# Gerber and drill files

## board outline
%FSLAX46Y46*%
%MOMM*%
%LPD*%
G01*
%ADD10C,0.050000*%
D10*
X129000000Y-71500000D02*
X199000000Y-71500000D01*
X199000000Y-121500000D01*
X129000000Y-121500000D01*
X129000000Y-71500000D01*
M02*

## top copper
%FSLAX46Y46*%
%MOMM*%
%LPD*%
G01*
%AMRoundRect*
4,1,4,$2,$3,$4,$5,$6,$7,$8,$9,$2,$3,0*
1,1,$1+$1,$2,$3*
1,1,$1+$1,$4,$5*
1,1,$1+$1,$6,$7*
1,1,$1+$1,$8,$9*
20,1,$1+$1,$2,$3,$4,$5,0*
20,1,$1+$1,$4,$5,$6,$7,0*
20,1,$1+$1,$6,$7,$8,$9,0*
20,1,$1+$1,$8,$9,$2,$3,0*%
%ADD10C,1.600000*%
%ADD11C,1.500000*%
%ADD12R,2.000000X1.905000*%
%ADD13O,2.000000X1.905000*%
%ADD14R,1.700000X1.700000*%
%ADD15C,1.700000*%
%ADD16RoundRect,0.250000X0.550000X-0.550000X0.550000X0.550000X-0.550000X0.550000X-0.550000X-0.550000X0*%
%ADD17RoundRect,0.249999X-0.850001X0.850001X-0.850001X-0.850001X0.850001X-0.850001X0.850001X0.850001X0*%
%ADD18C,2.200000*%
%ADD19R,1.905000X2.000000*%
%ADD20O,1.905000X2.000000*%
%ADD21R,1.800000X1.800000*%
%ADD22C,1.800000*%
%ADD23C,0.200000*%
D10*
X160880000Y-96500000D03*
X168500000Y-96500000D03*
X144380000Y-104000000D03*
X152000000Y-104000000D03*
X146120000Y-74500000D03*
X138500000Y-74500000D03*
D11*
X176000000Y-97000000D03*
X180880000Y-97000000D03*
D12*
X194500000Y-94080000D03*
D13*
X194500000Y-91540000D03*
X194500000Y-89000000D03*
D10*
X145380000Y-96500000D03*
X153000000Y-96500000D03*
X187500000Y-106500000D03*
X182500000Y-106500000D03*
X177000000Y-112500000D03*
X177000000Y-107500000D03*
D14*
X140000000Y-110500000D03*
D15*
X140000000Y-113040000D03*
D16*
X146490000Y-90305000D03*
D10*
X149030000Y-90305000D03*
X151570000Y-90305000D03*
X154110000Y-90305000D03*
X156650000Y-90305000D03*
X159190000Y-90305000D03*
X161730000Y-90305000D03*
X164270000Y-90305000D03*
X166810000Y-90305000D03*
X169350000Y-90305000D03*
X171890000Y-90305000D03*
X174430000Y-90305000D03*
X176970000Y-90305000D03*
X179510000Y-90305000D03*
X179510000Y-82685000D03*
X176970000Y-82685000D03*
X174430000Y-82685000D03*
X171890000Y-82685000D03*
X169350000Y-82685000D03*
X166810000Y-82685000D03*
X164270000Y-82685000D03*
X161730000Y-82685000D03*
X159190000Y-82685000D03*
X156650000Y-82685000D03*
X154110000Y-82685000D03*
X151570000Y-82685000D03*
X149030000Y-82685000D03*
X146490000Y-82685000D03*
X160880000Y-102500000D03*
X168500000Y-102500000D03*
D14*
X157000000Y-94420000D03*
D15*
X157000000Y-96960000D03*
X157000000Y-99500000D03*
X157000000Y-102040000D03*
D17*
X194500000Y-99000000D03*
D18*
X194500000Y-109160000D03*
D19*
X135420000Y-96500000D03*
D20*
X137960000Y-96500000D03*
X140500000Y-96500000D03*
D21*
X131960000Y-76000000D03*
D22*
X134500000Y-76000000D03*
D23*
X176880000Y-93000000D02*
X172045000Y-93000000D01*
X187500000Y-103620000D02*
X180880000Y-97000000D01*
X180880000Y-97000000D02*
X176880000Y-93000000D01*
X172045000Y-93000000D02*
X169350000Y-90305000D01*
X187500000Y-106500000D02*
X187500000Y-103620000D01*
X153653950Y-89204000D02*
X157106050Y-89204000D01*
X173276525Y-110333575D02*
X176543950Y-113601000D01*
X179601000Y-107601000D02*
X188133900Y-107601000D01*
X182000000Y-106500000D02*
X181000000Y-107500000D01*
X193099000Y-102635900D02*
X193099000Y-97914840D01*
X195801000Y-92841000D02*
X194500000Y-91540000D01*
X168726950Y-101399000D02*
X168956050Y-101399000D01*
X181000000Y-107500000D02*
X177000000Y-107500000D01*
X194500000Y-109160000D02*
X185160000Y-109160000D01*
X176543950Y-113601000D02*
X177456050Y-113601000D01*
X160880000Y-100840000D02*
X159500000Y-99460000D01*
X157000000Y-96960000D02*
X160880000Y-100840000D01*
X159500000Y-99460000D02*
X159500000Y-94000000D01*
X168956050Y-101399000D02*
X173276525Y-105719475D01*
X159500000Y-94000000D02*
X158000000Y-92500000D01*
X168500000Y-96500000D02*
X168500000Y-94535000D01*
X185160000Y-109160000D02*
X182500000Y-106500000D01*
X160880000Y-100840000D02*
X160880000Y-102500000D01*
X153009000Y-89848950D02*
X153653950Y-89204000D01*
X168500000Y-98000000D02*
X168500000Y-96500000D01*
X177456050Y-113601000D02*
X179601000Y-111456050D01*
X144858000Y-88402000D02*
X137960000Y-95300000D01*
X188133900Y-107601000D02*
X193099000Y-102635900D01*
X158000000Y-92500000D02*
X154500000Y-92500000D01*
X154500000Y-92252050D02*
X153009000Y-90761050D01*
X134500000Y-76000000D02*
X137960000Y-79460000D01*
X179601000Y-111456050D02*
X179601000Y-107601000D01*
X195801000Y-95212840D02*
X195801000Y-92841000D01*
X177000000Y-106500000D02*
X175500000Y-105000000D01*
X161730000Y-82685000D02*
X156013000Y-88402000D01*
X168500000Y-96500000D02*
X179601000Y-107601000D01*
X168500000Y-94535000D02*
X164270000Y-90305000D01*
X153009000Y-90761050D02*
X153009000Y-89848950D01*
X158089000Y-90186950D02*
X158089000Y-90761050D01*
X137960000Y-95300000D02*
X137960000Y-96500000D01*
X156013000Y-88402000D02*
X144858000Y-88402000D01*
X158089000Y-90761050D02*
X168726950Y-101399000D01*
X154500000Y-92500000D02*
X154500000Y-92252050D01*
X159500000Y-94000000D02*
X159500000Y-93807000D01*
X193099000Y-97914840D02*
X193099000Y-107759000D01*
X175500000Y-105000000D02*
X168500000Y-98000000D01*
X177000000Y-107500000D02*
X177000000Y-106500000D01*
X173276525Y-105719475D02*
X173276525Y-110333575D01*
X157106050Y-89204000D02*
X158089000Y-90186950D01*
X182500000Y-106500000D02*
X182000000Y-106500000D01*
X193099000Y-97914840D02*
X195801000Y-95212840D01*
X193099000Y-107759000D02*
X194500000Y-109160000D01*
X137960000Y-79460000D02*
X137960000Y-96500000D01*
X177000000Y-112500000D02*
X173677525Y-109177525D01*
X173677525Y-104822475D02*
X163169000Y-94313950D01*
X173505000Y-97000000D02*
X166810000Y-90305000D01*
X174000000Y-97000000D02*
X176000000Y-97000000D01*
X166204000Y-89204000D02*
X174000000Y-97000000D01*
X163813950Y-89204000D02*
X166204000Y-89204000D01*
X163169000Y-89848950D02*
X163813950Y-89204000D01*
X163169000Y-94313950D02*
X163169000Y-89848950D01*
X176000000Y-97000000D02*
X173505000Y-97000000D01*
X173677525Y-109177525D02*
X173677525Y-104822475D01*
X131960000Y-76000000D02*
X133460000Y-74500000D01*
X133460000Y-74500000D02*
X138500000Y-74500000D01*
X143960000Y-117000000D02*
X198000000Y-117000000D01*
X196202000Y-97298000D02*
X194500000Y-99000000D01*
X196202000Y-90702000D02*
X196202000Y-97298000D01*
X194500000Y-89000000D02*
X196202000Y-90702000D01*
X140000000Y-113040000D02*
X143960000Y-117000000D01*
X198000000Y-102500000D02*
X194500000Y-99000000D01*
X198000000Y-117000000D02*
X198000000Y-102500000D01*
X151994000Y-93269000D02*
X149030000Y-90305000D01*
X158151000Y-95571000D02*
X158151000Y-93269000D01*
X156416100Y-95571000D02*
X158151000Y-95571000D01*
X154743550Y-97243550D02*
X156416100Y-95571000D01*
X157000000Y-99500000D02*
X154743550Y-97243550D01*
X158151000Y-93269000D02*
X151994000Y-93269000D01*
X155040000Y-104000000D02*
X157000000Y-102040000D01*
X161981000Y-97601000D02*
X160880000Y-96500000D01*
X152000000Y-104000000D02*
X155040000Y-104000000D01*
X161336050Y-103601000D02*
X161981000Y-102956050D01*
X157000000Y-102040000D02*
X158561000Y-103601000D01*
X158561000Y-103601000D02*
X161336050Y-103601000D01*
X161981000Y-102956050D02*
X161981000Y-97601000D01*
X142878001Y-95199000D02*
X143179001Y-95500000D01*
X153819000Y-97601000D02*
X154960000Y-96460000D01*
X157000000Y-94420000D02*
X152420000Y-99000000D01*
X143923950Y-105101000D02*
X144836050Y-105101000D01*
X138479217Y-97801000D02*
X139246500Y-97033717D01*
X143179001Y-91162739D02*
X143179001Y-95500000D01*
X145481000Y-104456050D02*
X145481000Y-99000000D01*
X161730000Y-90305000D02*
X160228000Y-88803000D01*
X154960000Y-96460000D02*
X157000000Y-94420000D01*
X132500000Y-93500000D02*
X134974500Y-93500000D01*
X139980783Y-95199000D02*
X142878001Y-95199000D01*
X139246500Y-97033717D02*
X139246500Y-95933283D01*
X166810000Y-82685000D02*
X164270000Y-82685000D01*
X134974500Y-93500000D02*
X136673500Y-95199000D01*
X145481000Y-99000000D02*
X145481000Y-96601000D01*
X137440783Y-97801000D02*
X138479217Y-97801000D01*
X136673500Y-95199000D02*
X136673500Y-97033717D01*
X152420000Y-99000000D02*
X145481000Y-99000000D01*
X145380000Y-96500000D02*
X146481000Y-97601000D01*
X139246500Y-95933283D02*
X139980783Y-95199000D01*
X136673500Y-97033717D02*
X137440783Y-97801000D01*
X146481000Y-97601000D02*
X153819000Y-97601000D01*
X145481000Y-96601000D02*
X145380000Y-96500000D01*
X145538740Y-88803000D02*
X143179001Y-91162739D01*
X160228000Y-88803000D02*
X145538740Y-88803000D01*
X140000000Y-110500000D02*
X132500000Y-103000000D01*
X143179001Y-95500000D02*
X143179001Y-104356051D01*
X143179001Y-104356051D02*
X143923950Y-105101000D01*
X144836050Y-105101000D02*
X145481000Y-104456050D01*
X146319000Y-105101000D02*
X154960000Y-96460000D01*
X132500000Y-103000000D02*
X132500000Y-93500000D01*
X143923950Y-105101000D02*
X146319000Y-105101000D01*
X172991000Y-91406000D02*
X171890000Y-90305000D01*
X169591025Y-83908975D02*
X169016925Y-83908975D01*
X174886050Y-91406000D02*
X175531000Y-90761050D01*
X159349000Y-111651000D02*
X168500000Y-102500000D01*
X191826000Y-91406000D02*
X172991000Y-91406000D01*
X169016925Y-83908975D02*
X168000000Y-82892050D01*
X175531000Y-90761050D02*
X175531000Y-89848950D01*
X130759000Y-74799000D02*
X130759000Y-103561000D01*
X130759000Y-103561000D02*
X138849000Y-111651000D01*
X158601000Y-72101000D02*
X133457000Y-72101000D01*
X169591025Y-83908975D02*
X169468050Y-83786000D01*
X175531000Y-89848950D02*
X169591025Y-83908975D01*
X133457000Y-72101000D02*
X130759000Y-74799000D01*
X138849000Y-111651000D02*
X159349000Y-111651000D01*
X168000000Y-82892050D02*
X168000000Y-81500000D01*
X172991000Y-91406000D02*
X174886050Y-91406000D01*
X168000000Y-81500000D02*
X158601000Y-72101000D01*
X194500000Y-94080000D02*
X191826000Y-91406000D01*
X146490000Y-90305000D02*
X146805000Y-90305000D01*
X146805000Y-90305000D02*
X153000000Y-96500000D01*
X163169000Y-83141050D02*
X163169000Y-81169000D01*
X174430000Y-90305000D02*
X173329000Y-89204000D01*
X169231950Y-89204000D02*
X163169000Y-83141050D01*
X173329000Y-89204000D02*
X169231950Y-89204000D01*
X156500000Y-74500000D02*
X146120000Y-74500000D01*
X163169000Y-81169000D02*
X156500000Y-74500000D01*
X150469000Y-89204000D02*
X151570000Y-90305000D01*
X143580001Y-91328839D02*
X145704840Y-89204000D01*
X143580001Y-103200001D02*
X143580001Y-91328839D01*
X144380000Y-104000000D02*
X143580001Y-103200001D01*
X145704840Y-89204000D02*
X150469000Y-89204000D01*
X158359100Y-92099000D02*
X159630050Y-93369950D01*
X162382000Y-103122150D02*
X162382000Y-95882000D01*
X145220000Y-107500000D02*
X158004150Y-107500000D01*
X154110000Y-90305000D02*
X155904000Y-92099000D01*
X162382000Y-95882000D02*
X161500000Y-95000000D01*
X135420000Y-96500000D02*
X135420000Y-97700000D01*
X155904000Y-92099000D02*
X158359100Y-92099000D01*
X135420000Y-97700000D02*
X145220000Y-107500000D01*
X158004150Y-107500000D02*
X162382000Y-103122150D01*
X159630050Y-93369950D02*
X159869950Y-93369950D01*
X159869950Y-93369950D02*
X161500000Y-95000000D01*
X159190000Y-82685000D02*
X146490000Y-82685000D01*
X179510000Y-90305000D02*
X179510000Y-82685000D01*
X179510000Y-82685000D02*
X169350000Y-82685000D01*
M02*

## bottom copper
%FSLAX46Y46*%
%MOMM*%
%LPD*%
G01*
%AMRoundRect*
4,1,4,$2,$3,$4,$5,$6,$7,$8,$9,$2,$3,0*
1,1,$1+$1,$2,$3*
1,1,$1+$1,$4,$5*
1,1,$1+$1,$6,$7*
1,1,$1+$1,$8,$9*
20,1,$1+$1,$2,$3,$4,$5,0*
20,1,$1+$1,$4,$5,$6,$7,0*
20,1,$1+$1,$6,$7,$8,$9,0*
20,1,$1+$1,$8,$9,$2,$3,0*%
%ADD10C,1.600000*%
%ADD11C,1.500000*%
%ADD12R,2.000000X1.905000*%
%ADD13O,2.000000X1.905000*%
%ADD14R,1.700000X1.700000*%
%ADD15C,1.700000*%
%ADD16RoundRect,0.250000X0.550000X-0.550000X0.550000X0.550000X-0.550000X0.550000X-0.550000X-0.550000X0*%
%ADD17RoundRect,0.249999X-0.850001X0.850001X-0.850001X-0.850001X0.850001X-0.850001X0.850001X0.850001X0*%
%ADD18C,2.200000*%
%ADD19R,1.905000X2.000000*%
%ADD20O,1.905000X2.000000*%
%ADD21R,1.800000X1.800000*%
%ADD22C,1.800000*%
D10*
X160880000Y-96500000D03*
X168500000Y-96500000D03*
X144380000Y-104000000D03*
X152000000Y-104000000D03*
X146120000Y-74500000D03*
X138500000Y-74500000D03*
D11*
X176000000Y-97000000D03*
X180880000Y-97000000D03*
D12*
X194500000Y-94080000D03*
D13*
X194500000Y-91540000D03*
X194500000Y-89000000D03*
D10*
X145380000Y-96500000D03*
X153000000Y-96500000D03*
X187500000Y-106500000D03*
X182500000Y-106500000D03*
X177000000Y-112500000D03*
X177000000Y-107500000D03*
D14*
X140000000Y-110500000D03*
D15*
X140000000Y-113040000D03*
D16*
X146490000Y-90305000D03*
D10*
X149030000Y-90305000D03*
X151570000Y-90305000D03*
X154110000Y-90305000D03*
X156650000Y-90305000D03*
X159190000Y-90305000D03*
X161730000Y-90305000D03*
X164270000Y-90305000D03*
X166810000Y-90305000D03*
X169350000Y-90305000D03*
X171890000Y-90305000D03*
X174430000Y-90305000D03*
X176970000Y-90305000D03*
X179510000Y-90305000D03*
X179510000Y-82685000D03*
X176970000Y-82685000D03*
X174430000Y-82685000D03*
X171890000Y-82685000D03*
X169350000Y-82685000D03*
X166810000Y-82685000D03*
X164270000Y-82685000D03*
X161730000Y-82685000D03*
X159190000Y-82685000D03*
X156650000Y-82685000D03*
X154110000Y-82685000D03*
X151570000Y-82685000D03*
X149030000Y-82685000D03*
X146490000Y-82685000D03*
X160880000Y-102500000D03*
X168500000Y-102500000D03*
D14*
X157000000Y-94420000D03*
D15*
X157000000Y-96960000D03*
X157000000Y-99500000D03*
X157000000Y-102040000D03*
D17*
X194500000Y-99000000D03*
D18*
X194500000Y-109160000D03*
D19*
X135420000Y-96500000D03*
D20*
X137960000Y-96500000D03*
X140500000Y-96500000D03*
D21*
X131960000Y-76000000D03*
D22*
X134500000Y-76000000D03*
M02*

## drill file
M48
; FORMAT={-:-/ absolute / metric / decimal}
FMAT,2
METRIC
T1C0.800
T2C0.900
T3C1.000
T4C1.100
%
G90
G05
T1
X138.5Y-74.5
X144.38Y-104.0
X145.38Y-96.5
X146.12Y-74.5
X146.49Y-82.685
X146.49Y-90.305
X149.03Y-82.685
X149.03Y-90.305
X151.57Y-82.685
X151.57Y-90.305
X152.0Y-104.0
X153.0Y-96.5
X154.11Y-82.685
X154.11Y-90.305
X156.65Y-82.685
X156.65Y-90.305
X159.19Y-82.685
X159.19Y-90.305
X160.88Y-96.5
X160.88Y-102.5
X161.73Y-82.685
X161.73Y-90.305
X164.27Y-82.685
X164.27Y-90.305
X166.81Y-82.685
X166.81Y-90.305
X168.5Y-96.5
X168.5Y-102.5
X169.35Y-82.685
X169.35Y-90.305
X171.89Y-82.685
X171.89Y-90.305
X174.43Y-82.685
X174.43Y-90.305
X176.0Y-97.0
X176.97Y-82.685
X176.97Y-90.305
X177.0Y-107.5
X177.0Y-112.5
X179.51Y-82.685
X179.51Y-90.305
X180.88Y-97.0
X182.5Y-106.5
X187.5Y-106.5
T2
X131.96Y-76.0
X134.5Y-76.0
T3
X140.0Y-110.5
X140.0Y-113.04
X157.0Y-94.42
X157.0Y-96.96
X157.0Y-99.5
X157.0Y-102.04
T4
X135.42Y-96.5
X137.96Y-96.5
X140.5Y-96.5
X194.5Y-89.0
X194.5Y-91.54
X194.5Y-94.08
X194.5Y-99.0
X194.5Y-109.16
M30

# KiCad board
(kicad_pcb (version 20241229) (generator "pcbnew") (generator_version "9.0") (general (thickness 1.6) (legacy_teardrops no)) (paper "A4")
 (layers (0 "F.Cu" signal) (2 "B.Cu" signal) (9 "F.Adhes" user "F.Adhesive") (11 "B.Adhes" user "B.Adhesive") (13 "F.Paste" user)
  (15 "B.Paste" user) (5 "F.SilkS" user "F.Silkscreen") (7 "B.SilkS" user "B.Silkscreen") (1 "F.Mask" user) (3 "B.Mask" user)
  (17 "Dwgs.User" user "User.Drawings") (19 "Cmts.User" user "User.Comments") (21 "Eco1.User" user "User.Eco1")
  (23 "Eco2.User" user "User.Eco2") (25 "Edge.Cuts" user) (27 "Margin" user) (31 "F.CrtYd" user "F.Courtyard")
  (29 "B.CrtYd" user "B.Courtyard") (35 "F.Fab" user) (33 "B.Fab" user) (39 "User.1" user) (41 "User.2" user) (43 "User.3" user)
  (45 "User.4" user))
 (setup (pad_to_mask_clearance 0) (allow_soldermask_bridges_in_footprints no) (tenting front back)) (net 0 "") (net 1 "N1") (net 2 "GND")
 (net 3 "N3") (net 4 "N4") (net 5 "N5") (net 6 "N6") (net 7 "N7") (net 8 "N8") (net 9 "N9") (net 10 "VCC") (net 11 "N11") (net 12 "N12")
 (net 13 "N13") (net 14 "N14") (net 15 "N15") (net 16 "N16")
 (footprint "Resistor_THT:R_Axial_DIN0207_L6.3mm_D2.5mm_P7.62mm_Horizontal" (layer "F.Cu") (at 160.88 96.5)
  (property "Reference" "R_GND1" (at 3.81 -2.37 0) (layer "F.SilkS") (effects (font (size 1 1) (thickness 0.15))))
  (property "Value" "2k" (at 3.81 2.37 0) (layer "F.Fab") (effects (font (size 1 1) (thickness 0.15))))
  (pad "1" thru_hole circle (at 0 0) (size 1.6 1.6) (drill 0.8) (layers "*.Cu" "*.Mask") (remove_unused_layers no) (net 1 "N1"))
  (pad "2" thru_hole circle (at 7.62 0) (size 1.6 1.6) (drill 0.8) (layers "*.Cu" "*.Mask") (remove_unused_layers no) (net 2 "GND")))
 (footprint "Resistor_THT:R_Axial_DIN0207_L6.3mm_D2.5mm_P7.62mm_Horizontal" (layer "F.Cu") (at 144.38 104)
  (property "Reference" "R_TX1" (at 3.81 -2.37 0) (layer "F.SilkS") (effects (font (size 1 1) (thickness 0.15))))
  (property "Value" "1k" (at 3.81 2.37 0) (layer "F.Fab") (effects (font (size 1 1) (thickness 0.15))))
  (pad "1" thru_hole circle (at 0 0) (size 1.6 1.6) (drill 0.8) (layers "*.Cu" "*.Mask") (remove_unused_layers no) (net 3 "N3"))
  (pad "2" thru_hole circle (at 7.62 0) (size 1.6 1.6) (drill 0.8) (layers "*.Cu" "*.Mask") (remove_unused_layers no) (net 1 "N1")))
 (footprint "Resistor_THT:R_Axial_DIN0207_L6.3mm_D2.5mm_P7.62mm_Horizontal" (layer "F.Cu") (at 146.12 74.5 180)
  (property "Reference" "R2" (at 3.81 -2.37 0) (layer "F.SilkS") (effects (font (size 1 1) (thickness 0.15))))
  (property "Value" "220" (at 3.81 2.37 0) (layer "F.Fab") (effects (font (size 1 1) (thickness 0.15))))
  (pad "1" thru_hole circle (at 0 0 180) (size 1.6 1.6) (drill 0.8) (layers "*.Cu" "*.Mask") (remove_unused_layers no) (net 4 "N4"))
  (pad "2" thru_hole circle (at 7.62 0 180) (size 1.6 1.6) (drill 0.8) (layers "*.Cu" "*.Mask") (remove_unused_layers no) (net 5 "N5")))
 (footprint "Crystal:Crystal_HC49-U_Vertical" (layer "F.Cu") (at 176 97)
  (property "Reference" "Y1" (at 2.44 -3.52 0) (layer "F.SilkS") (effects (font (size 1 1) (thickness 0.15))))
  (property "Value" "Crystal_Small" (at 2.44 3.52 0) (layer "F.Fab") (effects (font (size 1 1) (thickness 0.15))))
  (pad "1" thru_hole circle (at 0 0) (size 1.5 1.5) (drill 0.8) (layers "*.Cu" "*.Mask") (remove_unused_layers no) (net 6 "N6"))
  (pad "2" thru_hole circle (at 4.88 0) (size 1.5 1.5) (drill 0.8) (layers "*.Cu" "*.Mask") (remove_unused_layers no) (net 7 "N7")))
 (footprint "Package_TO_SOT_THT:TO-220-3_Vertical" (layer "F.Cu") (at 194.5 94.08 90)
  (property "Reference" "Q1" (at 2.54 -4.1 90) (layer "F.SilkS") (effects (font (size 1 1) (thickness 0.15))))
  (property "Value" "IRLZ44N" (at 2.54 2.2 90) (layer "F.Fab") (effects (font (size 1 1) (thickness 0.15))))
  (pad "1" thru_hole rect (at 0 0 90) (size 1.905 2) (drill 1.1) (layers "*.Cu" "*.Mask") (remove_unused_layers no) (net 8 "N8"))
  (pad "2" thru_hole oval (at 2.54 0 90) (size 1.905 2) (drill 1.1) (layers "*.Cu" "*.Mask") (remove_unused_layers no) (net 2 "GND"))
  (pad "3" thru_hole oval (at 5.08 0 90) (size 1.905 2) (drill 1.1) (layers "*.Cu" "*.Mask") (remove_unused_layers no) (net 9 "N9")))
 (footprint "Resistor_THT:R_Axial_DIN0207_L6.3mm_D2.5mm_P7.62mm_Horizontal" (layer "F.Cu") (at 145.38 96.5)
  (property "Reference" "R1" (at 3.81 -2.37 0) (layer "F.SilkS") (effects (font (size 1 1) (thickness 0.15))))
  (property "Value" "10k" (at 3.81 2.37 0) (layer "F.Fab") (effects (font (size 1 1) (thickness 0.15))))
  (pad "1" thru_hole circle (at 0 0) (size 1.6 1.6) (drill 0.8) (layers "*.Cu" "*.Mask") (remove_unused_layers no) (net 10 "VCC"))
  (pad "2" thru_hole circle (at 7.62 0) (size 1.6 1.6) (drill 0.8) (layers "*.Cu" "*.Mask") (remove_unused_layers no) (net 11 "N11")))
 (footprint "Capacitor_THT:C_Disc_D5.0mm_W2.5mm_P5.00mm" (layer "F.Cu") (at 187.5 106.5 180)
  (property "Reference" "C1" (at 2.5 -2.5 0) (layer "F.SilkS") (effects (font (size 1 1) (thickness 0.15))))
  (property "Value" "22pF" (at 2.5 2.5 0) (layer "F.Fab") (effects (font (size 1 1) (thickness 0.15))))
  (pad "1" thru_hole circle (at 0 0 180) (size 1.6 1.6) (drill 0.8) (layers "*.Cu" "*.Mask") (remove_unused_layers no) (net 7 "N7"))
  (pad "2" thru_hole circle (at 5 0 180) (size 1.6 1.6) (drill 0.8) (layers "*.Cu" "*.Mask") (remove_unused_layers no) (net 2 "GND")))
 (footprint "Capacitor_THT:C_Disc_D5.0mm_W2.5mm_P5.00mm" (layer "F.Cu") (at 177 112.5 90)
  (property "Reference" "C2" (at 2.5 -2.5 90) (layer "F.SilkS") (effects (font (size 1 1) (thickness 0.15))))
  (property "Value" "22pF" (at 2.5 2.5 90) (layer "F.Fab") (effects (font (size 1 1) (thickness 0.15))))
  (pad "1" thru_hole circle (at 0 0 90) (size 1.6 1.6) (drill 0.8) (layers "*.Cu" "*.Mask") (remove_unused_layers no) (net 6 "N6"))
  (pad "2" thru_hole circle (at 5 0 90) (size 1.6 1.6) (drill 0.8) (layers "*.Cu" "*.Mask") (remove_unused_layers no) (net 2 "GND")))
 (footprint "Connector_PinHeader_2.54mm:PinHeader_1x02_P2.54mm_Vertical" (layer "F.Cu") (at 140 110.5)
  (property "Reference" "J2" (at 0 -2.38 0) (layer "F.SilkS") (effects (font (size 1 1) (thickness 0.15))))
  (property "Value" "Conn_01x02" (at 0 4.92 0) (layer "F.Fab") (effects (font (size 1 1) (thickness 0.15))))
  (pad "1" thru_hole rect (at 0 0) (size 1.7 1.7) (drill 1) (layers "*.Cu" "*.Mask") (remove_unused_layers no) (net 10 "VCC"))
  (pad "2" thru_hole circle (at 0 2.54) (size 1.7 1.7) (drill 1) (layers "*.Cu" "*.Mask") (remove_unused_layers no) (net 9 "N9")))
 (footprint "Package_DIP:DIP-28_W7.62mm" (layer "F.Cu") (at 146.49 90.305 90)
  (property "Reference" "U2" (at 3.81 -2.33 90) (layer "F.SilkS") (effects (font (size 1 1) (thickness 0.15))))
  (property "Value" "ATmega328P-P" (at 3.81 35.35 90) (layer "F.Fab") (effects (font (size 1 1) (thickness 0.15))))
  (pad "1" thru_hole roundrect (at 0 0 90) (size 1.6 1.6) (drill 0.8) (layers "*.Cu" "*.Mask") (remove_unused_layers no)
   (roundrect_rratio 0.15625) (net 11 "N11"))
  (pad "2" thru_hole circle (at 0 2.54 90) (size 1.6 1.6) (drill 0.8) (layers "*.Cu" "*.Mask") (remove_unused_layers no) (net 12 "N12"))
  (pad "3" thru_hole circle (at 0 5.08 90) (size 1.6 1.6) (drill 0.8) (layers "*.Cu" "*.Mask") (remove_unused_layers no) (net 3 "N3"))
  (pad "4" thru_hole circle (at 0 7.62 90) (size 1.6 1.6) (drill 0.8) (layers "*.Cu" "*.Mask") (remove_unused_layers no) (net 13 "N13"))
  (pad "5" thru_hole circle (at 0 10.16 90) (size 1.6 1.6) (drill 0.8) (layers "*.Cu" "*.Mask") (remove_unused_layers no) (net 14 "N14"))
  (pad "6" thru_hole circle (at 0 12.7 90) (size 1.6 1.6) (drill 0.8) (layers "*.Cu" "*.Mask") (remove_unused_layers no) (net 14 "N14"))
  (pad "7" thru_hole circle (at 0 15.24 90) (size 1.6 1.6) (drill 0.8) (layers "*.Cu" "*.Mask") (remove_unused_layers no) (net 10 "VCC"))
  (pad "8" thru_hole circle (at 0 17.78 90) (size 1.6 1.6) (drill 0.8) (layers "*.Cu" "*.Mask") (remove_unused_layers no) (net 2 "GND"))
  (pad "9" thru_hole circle (at 0 20.32 90) (size 1.6 1.6) (drill 0.8) (layers "*.Cu" "*.Mask") (remove_unused_layers no) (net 6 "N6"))
  (pad "10" thru_hole circle (at 0 22.86 90) (size 1.6 1.6) (drill 0.8) (layers "*.Cu" "*.Mask") (remove_unused_layers no) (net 7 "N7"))
  (pad "11" thru_hole circle (at 0 25.4 90) (size 1.6 1.6) (drill 0.8) (layers "*.Cu" "*.Mask") (remove_unused_layers no) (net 8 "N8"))
  (pad "12" thru_hole circle (at 0 27.94 90) (size 1.6 1.6) (drill 0.8) (layers "*.Cu" "*.Mask") (remove_unused_layers no) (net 4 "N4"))
  (pad "13" thru_hole circle (at 0 30.48 90) (size 1.6 1.6) (drill 0.8) (layers "*.Cu" "*.Mask") (remove_unused_layers no) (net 14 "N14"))
  (pad "14" thru_hole circle (at 0 33.02 90) (size 1.6 1.6) (drill 0.8) (layers "*.Cu" "*.Mask") (remove_unused_layers no) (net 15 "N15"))
  (pad "15" thru_hole circle (at 7.62 33.02 90) (size 1.6 1.6) (drill 0.8) (layers "*.Cu" "*.Mask") (remove_unused_layers no) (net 15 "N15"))
  (pad "16" thru_hole circle (at 7.62 30.48 90) (size 1.6 1.6) (drill 0.8) (layers "*.Cu" "*.Mask") (remove_unused_layers no) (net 15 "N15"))
  (pad "17" thru_hole circle (at 7.62 27.94 90) (size 1.6 1.6) (drill 0.8) (layers "*.Cu" "*.Mask") (remove_unused_layers no) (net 15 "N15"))
  (pad "18" thru_hole circle (at 7.62 25.4 90) (size 1.6 1.6) (drill 0.8) (layers "*.Cu" "*.Mask") (remove_unused_layers no) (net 15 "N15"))
  (pad "19" thru_hole circle (at 7.62 22.86 90) (size 1.6 1.6) (drill 0.8) (layers "*.Cu" "*.Mask") (remove_unused_layers no) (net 15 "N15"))
  (pad "20" thru_hole circle (at 7.62 20.32 90) (size 1.6 1.6) (drill 0.8) (layers "*.Cu" "*.Mask") (remove_unused_layers no) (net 10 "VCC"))
  (pad "21" thru_hole circle (at 7.62 17.78 90) (size 1.6 1.6) (drill 0.8) (layers "*.Cu" "*.Mask") (remove_unused_layers no) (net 10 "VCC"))
  (pad "22" thru_hole circle (at 7.62 15.24 90) (size 1.6 1.6) (drill 0.8) (layers "*.Cu" "*.Mask") (remove_unused_layers no) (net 2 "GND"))
  (pad "23" thru_hole circle (at 7.62 12.7 90) (size 1.6 1.6) (drill 0.8) (layers "*.Cu" "*.Mask") (remove_unused_layers no) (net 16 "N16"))
  (pad "24" thru_hole circle (at 7.62 10.16 90) (size 1.6 1.6) (drill 0.8) (layers "*.Cu" "*.Mask") (remove_unused_layers no) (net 16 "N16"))
  (pad "25" thru_hole circle (at 7.62 7.62 90) (size 1.6 1.6) (drill 0.8) (layers "*.Cu" "*.Mask") (remove_unused_layers no) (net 16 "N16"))
  (pad "26" thru_hole circle (at 7.62 5.08 90) (size 1.6 1.6) (drill 0.8) (layers "*.Cu" "*.Mask") (remove_unused_layers no) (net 16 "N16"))
  (pad "27" thru_hole circle (at 7.62 2.54 90) (size 1.6 1.6) (drill 0.8) (layers "*.Cu" "*.Mask") (remove_unused_layers no) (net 16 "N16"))
  (pad "28" thru_hole circle (at 7.62 0 90) (size 1.6 1.6) (drill 0.8) (layers "*.Cu" "*.Mask") (remove_unused_layers no) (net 16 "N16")))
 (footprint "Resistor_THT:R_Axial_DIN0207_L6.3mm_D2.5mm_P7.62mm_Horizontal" (layer "F.Cu") (at 160.88 102.5)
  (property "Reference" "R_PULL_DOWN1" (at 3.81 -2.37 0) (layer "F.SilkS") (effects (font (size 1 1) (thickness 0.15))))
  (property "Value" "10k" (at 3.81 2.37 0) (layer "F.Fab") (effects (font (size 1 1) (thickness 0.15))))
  (pad "1" thru_hole circle (at 0 0) (size 1.6 1.6) (drill 0.8) (layers "*.Cu" "*.Mask") (remove_unused_layers no) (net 2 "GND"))
  (pad "2" thru_hole circle (at 7.62 0) (size 1.6 1.6) (drill 0.8) (layers "*.Cu" "*.Mask") (remove_unused_layers no) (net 8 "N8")))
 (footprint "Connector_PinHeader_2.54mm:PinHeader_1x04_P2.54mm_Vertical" (layer "F.Cu") (at 157 94.42)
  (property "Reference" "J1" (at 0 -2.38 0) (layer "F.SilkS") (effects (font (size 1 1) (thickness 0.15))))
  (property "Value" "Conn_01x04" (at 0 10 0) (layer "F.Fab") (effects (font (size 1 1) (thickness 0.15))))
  (pad "1" thru_hole rect (at 0 0) (size 1.7 1.7) (drill 1) (layers "*.Cu" "*.Mask") (remove_unused_layers no) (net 10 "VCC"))
  (pad "2" thru_hole circle (at 0 2.54) (size 1.7 1.7) (drill 1) (layers "*.Cu" "*.Mask") (remove_unused_layers no) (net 2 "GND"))
  (pad "3" thru_hole circle (at 0 5.08) (size 1.7 1.7) (drill 1) (layers "*.Cu" "*.Mask") (remove_unused_layers no) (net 12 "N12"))
  (pad "4" thru_hole circle (at 0 7.62) (size 1.7 1.7) (drill 1) (layers "*.Cu" "*.Mask") (remove_unused_layers no) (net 1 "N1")))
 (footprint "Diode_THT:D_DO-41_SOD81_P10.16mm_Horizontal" (layer "F.Cu") (at 194.5 99 -90)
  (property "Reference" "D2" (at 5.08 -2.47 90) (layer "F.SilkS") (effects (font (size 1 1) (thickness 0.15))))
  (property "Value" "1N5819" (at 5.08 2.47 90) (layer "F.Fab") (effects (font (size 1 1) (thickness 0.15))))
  (pad "1" thru_hole roundrect (at 0 0 270) (size 2.2 2.2) (drill 1.1) (layers "*.Cu" "*.Mask") (remove_unused_layers no)
   (roundrect_rratio 0.113636) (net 9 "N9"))
  (pad "2" thru_hole circle (at 10.16 0 270) (size 2.2 2.2) (drill 1.1) (layers "*.Cu" "*.Mask") (remove_unused_layers no) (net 2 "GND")))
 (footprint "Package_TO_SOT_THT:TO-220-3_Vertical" (layer "F.Cu") (at 135.42 96.5)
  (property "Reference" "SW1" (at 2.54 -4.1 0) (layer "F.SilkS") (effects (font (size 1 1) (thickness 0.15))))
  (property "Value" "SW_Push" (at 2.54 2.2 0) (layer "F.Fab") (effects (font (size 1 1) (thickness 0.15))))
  (pad "1" thru_hole rect (at 0 0) (size 1.905 2) (drill 1.1) (layers "*.Cu" "*.Mask") (remove_unused_layers no) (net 13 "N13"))
  (pad "2" thru_hole oval (at 2.54 0) (size 1.905 2) (drill 1.1) (layers "*.Cu" "*.Mask") (remove_unused_layers no) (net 2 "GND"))
  (pad "3" thru_hole oval (at 5.08 0) (size 1.905 2) (drill 1.1) (layers "*.Cu" "*.Mask") (remove_unused_layers no)))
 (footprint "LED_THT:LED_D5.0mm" (layer "F.Cu") (at 131.96 76)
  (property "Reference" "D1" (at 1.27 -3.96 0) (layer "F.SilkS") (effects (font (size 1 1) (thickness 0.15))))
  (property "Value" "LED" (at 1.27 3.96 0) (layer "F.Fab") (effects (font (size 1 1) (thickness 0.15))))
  (pad "1" thru_hole rect (at 0 0) (size 1.8 1.8) (drill 0.9) (layers "*.Cu" "*.Mask") (remove_unused_layers no) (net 5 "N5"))
  (pad "2" thru_hole circle (at 2.54 0) (size 1.8 1.8) (drill 0.9) (layers "*.Cu" "*.Mask") (remove_unused_layers no) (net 2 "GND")))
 (gr_rect (start 129 71.5) (end 199 121.5) (stroke (width 0.05) (type default)) (fill no) (layer "Edge.Cuts"))
 (segment (start 176.88 93) (end 172.045 93) (width 0.2) (layer "F.Cu") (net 7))
 (segment (start 187.5 103.62) (end 180.88 97) (width 0.2) (layer "F.Cu") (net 7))
 (segment (start 180.88 97) (end 176.88 93) (width 0.2) (layer "F.Cu") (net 7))
 (segment (start 172.045 93) (end 169.35 90.305) (width 0.2) (layer "F.Cu") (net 7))
 (segment (start 187.5 106.5) (end 187.5 103.62) (width 0.2) (layer "F.Cu") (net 7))
 (segment (start 153.65395 89.204) (end 157.10605 89.204) (width 0.2) (layer "F.Cu") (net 2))
 (segment (start 173.276525 110.333575) (end 176.54395 113.601) (width 0.2) (layer "F.Cu") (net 2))
 (segment (start 179.601 107.601) (end 188.1339 107.601) (width 0.2) (layer "F.Cu") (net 2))
 (segment (start 182 106.5) (end 181 107.5) (width 0.2) (layer "F.Cu") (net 2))
 (segment (start 193.099 102.6359) (end 193.099 97.91484) (width 0.2) (layer "F.Cu") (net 2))
 (segment (start 195.801 92.841) (end 194.5 91.54) (width 0.2) (layer "F.Cu") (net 2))
 (segment (start 168.72695 101.399) (end 168.95605 101.399) (width 0.2) (layer "F.Cu") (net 2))
 (segment (start 181 107.5) (end 177 107.5) (width 0.2) (layer "F.Cu") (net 2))
 (segment (start 194.5 109.16) (end 185.16 109.16) (width 0.2) (layer "F.Cu") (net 2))
 (segment (start 176.54395 113.601) (end 177.45605 113.601) (width 0.2) (layer "F.Cu") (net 2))
 (segment (start 160.88 100.84) (end 159.5 99.46) (width 0.2) (layer "F.Cu") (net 2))
 (segment (start 157 96.96) (end 160.88 100.84) (width 0.2) (layer "F.Cu") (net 2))
 (segment (start 159.5 99.46) (end 159.5 94) (width 0.2) (layer "F.Cu") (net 2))
 (segment (start 168.95605 101.399) (end 173.276525 105.719475) (width 0.2) (layer "F.Cu") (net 2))
 (segment (start 159.5 94) (end 158 92.5) (width 0.2) (layer "F.Cu") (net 2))
 (segment (start 168.5 96.5) (end 168.5 94.535) (width 0.2) (layer "F.Cu") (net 2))
 (segment (start 185.16 109.16) (end 182.5 106.5) (width 0.2) (layer "F.Cu") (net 2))
 (segment (start 160.88 100.84) (end 160.88 102.5) (width 0.2) (layer "F.Cu") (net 2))
 (segment (start 153.009 89.84895) (end 153.65395 89.204) (width 0.2) (layer "F.Cu") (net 2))
 (segment (start 168.5 98) (end 168.5 96.5) (width 0.2) (layer "F.Cu") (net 2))
 (segment (start 177.45605 113.601) (end 179.601 111.45605) (width 0.2) (layer "F.Cu") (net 2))
 (segment (start 144.858 88.402) (end 137.96 95.3) (width 0.2) (layer "F.Cu") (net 2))
 (segment (start 188.1339 107.601) (end 193.099 102.6359) (width 0.2) (layer "F.Cu") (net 2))
 (segment (start 158 92.5) (end 154.5 92.5) (width 0.2) (layer "F.Cu") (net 2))
 (segment (start 154.5 92.25205) (end 153.009 90.76105) (width 0.2) (layer "F.Cu") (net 2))
 (segment (start 134.5 76) (end 137.96 79.46) (width 0.2) (layer "F.Cu") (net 2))
 (segment (start 179.601 111.45605) (end 179.601 107.601) (width 0.2) (layer "F.Cu") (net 2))
 (segment (start 195.801 95.21284) (end 195.801 92.841) (width 0.2) (layer "F.Cu") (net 2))
 (segment (start 177 106.5) (end 175.5 105) (width 0.2) (layer "F.Cu") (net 2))
 (segment (start 161.73 82.685) (end 156.013 88.402) (width 0.2) (layer "F.Cu") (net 2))
 (segment (start 168.5 96.5) (end 179.601 107.601) (width 0.2) (layer "F.Cu") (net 2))
 (segment (start 168.5 94.535) (end 164.27 90.305) (width 0.2) (layer "F.Cu") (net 2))
 (segment (start 153.009 90.76105) (end 153.009 89.84895) (width 0.2) (layer "F.Cu") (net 2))
 (segment (start 158.089 90.18695) (end 158.089 90.76105) (width 0.2) (layer "F.Cu") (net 2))
 (segment (start 137.96 95.3) (end 137.96 96.5) (width 0.2) (layer "F.Cu") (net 2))
 (segment (start 156.013 88.402) (end 144.858 88.402) (width 0.2) (layer "F.Cu") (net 2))
 (segment (start 158.089 90.76105) (end 168.72695 101.399) (width 0.2) (layer "F.Cu") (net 2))
 (segment (start 154.5 92.5) (end 154.5 92.25205) (width 0.2) (layer "F.Cu") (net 2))
 (segment (start 159.5 94) (end 159.5 93.807) (width 0.2) (layer "F.Cu") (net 2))
 (segment (start 193.099 97.91484) (end 193.099 107.759) (width 0.2) (layer "F.Cu") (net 2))
 (segment (start 175.5 105) (end 168.5 98) (width 0.2) (layer "F.Cu") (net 2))
 (segment (start 177 107.5) (end 177 106.5) (width 0.2) (layer "F.Cu") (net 2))
 (segment (start 173.276525 105.719475) (end 173.276525 110.333575) (width 0.2) (layer "F.Cu") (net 2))
 (segment (start 157.10605 89.204) (end 158.089 90.18695) (width 0.2) (layer "F.Cu") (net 2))
 (segment (start 182.5 106.5) (end 182 106.5) (width 0.2) (layer "F.Cu") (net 2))
 (segment (start 193.099 97.91484) (end 195.801 95.21284) (width 0.2) (layer "F.Cu") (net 2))
 (segment (start 193.099 107.759) (end 194.5 109.16) (width 0.2) (layer "F.Cu") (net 2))
 (segment (start 137.96 79.46) (end 137.96 96.5) (width 0.2) (layer "F.Cu") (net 2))
 (segment (start 177 112.5) (end 173.677525 109.177525) (width 0.2) (layer "F.Cu") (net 6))
 (segment (start 173.677525 104.822475) (end 163.169 94.31395) (width 0.2) (layer "F.Cu") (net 6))
 (segment (start 173.505 97) (end 166.81 90.305) (width 0.2) (layer "F.Cu") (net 6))
 (segment (start 174 97) (end 176 97) (width 0.2) (layer "F.Cu") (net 6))
 (segment (start 166.204 89.204) (end 174 97) (width 0.2) (layer "F.Cu") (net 6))
 (segment (start 163.81395 89.204) (end 166.204 89.204) (width 0.2) (layer "F.Cu") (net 6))
 (segment (start 163.169 89.84895) (end 163.81395 89.204) (width 0.2) (layer "F.Cu") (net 6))
 (segment (start 163.169 94.31395) (end 163.169 89.84895) (width 0.2) (layer "F.Cu") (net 6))
 (segment (start 176 97) (end 173.505 97) (width 0.2) (layer "F.Cu") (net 6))
 (segment (start 173.677525 109.177525) (end 173.677525 104.822475) (width 0.2) (layer "F.Cu") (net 6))
 (segment (start 131.96 76) (end 133.46 74.5) (width 0.2) (layer "F.Cu") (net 5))
 (segment (start 133.46 74.5) (end 138.5 74.5) (width 0.2) (layer "F.Cu") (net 5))
 (segment (start 143.96 117) (end 198 117) (width 0.2) (layer "F.Cu") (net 9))
 (segment (start 196.202 97.298) (end 194.5 99) (width 0.2) (layer "F.Cu") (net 9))
 (segment (start 196.202 90.702) (end 196.202 97.298) (width 0.2) (layer "F.Cu") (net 9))
 (segment (start 194.5 89) (end 196.202 90.702) (width 0.2) (layer "F.Cu") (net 9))
 (segment (start 140 113.04) (end 143.96 117) (width 0.2) (layer "F.Cu") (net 9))
 (segment (start 198 102.5) (end 194.5 99) (width 0.2) (layer "F.Cu") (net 9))
 (segment (start 198 117) (end 198 102.5) (width 0.2) (layer "F.Cu") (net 9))
 (segment (start 151.994 93.269) (end 149.03 90.305) (width 0.2) (layer "F.Cu") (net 12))
 (segment (start 158.151 95.571) (end 158.151 93.269) (width 0.2) (layer "F.Cu") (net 12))
 (segment (start 156.4161 95.571) (end 158.151 95.571) (width 0.2) (layer "F.Cu") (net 12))
 (segment (start 154.74355 97.24355) (end 156.4161 95.571) (width 0.2) (layer "F.Cu") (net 12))
 (segment (start 157 99.5) (end 154.74355 97.24355) (width 0.2) (layer "F.Cu") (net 12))
 (segment (start 158.151 93.269) (end 151.994 93.269) (width 0.2) (layer "F.Cu") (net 12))
 (segment (start 155.04 104) (end 157 102.04) (width 0.2) (layer "F.Cu") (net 1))
 (segment (start 161.981 97.601) (end 160.88 96.5) (width 0.2) (layer "F.Cu") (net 1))
 (segment (start 152 104) (end 155.04 104) (width 0.2) (layer "F.Cu") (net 1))
 (segment (start 161.33605 103.601) (end 161.981 102.95605) (width 0.2) (layer "F.Cu") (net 1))
 (segment (start 157 102.04) (end 158.561 103.601) (width 0.2) (layer "F.Cu") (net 1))
 (segment (start 158.561 103.601) (end 161.33605 103.601) (width 0.2) (layer "F.Cu") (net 1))
 (segment (start 161.981 102.95605) (end 161.981 97.601) (width 0.2) (layer "F.Cu") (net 1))
 (segment (start 142.878001 95.199) (end 143.179001 95.5) (width 0.2) (layer "F.Cu") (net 10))
 (segment (start 153.819 97.601) (end 154.96 96.46) (width 0.2) (layer "F.Cu") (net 10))
 (segment (start 157 94.42) (end 152.42 99) (width 0.2) (layer "F.Cu") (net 10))
 (segment (start 143.92395 105.101) (end 144.83605 105.101) (width 0.2) (layer "F.Cu") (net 10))
 (segment (start 138.479217 97.801) (end 139.2465 97.033717) (width 0.2) (layer "F.Cu") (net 10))
 (segment (start 143.179001 91.162739) (end 143.179001 95.5) (width 0.2) (layer "F.Cu") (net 10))
 (segment (start 145.481 104.45605) (end 145.481 99) (width 0.2) (layer "F.Cu") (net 10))
 (segment (start 161.73 90.305) (end 160.228 88.803) (width 0.2) (layer "F.Cu") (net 10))
 (segment (start 154.96 96.46) (end 157 94.42) (width 0.2) (layer "F.Cu") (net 10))
 (segment (start 132.5 93.5) (end 134.9745 93.5) (width 0.2) (layer "F.Cu") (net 10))
 (segment (start 139.980783 95.199) (end 142.878001 95.199) (width 0.2) (layer "F.Cu") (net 10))
 (segment (start 139.2465 97.033717) (end 139.2465 95.933283) (width 0.2) (layer "F.Cu") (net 10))
 (segment (start 166.81 82.685) (end 164.27 82.685) (width 0.2) (layer "F.Cu") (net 10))
 (segment (start 134.9745 93.5) (end 136.6735 95.199) (width 0.2) (layer "F.Cu") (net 10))
 (segment (start 145.481 99) (end 145.481 96.601) (width 0.2) (layer "F.Cu") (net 10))
 (segment (start 137.440783 97.801) (end 138.479217 97.801) (width 0.2) (layer "F.Cu") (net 10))
 (segment (start 136.6735 95.199) (end 136.6735 97.033717) (width 0.2) (layer "F.Cu") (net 10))
 (segment (start 152.42 99) (end 145.481 99) (width 0.2) (layer "F.Cu") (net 10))
 (segment (start 145.38 96.5) (end 146.481 97.601) (width 0.2) (layer "F.Cu") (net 10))
 (segment (start 139.2465 95.933283) (end 139.980783 95.199) (width 0.2) (layer "F.Cu") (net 10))
 (segment (start 136.6735 97.033717) (end 137.440783 97.801) (width 0.2) (layer "F.Cu") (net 10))
 (segment (start 146.481 97.601) (end 153.819 97.601) (width 0.2) (layer "F.Cu") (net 10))
 (segment (start 145.481 96.601) (end 145.38 96.5) (width 0.2) (layer "F.Cu") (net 10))
 (segment (start 145.53874 88.803) (end 143.179001 91.162739) (width 0.2) (layer "F.Cu") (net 10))
 (segment (start 160.228 88.803) (end 145.53874 88.803) (width 0.2) (layer "F.Cu") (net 10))
 (segment (start 140 110.5) (end 132.5 103) (width 0.2) (layer "F.Cu") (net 10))
 (segment (start 143.179001 95.5) (end 143.179001 104.356051) (width 0.2) (layer "F.Cu") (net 10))
 (segment (start 143.179001 104.356051) (end 143.92395 105.101) (width 0.2) (layer "F.Cu") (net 10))
 (segment (start 144.83605 105.101) (end 145.481 104.45605) (width 0.2) (layer "F.Cu") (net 10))
 (segment (start 146.319 105.101) (end 154.96 96.46) (width 0.2) (layer "F.Cu") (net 10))
 (segment (start 132.5 103) (end 132.5 93.5) (width 0.2) (layer "F.Cu") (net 10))
 (segment (start 143.92395 105.101) (end 146.319 105.101) (width 0.2) (layer "F.Cu") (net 10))
 (segment (start 172.991 91.406) (end 171.89 90.305) (width 0.2) (layer "F.Cu") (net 8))
 (segment (start 169.591025 83.908975) (end 169.016925 83.908975) (width 0.2) (layer "F.Cu") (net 8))
 (segment (start 174.88605 91.406) (end 175.531 90.76105) (width 0.2) (layer "F.Cu") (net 8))
 (segment (start 159.349 111.651) (end 168.5 102.5) (width 0.2) (layer "F.Cu") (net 8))
 (segment (start 191.826 91.406) (end 172.991 91.406) (width 0.2) (layer "F.Cu") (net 8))
 (segment (start 169.016925 83.908975) (end 168 82.89205) (width 0.2) (layer "F.Cu") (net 8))
 (segment (start 175.531 90.76105) (end 175.531 89.84895) (width 0.2) (layer "F.Cu") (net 8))
 (segment (start 130.759 74.799) (end 130.759 103.561) (width 0.2) (layer "F.Cu") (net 8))
 (segment (start 130.759 103.561) (end 138.849 111.651) (width 0.2) (layer "F.Cu") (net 8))
 (segment (start 158.601 72.101) (end 133.457 72.101) (width 0.2) (layer "F.Cu") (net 8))
 (segment (start 169.591025 83.908975) (end 169.46805 83.786) (width 0.2) (layer "F.Cu") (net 8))
 (segment (start 175.531 89.84895) (end 169.591025 83.908975) (width 0.2) (layer "F.Cu") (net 8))
 (segment (start 133.457 72.101) (end 130.759 74.799) (width 0.2) (layer "F.Cu") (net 8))
 (segment (start 138.849 111.651) (end 159.349 111.651) (width 0.2) (layer "F.Cu") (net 8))
 (segment (start 168 82.89205) (end 168 81.5) (width 0.2) (layer "F.Cu") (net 8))
 (segment (start 172.991 91.406) (end 174.88605 91.406) (width 0.2) (layer "F.Cu") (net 8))
 (segment (start 168 81.5) (end 158.601 72.101) (width 0.2) (layer "F.Cu") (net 8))
 (segment (start 194.5 94.08) (end 191.826 91.406) (width 0.2) (layer "F.Cu") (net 8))
 (segment (start 146.49 90.305) (end 146.805 90.305) (width 0.2) (layer "F.Cu") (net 11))
 (segment (start 146.805 90.305) (end 153 96.5) (width 0.2) (layer "F.Cu") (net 11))
 (segment (start 163.169 83.14105) (end 163.169 81.169) (width 0.2) (layer "F.Cu") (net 4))
 (segment (start 174.43 90.305) (end 173.329 89.204) (width 0.2) (layer "F.Cu") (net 4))
 (segment (start 169.23195 89.204) (end 163.169 83.14105) (width 0.2) (layer "F.Cu") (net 4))
 (segment (start 173.329 89.204) (end 169.23195 89.204) (width 0.2) (layer "F.Cu") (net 4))
 (segment (start 156.5 74.5) (end 146.12 74.5) (width 0.2) (layer "F.Cu") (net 4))
 (segment (start 163.169 81.169) (end 156.5 74.5) (width 0.2) (layer "F.Cu") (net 4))
 (segment (start 150.469 89.204) (end 151.57 90.305) (width 0.2) (layer "F.Cu") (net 3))
 (segment (start 143.580001 91.328839) (end 145.70484 89.204) (width 0.2) (layer "F.Cu") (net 3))
 (segment (start 143.580001 103.200001) (end 143.580001 91.328839) (width 0.2) (layer "F.Cu") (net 3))
 (segment (start 144.38 104) (end 143.580001 103.200001) (width 0.2) (layer "F.Cu") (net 3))
 (segment (start 145.70484 89.204) (end 150.469 89.204) (width 0.2) (layer "F.Cu") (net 3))
 (segment (start 158.3591 92.099) (end 159.63005 93.36995) (width 0.2) (layer "F.Cu") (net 13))
 (segment (start 162.382 103.12215) (end 162.382 95.882) (width 0.2) (layer "F.Cu") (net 13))
 (segment (start 145.22 107.5) (end 158.00415 107.5) (width 0.2) (layer "F.Cu") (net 13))
 (segment (start 154.11 90.305) (end 155.904 92.099) (width 0.2) (layer "F.Cu") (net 13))
 (segment (start 162.382 95.882) (end 161.5 95) (width 0.2) (layer "F.Cu") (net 13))
 (segment (start 135.42 96.5) (end 135.42 97.7) (width 0.2) (layer "F.Cu") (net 13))
 (segment (start 155.904 92.099) (end 158.3591 92.099) (width 0.2) (layer "F.Cu") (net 13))
 (segment (start 135.42 97.7) (end 145.22 107.5) (width 0.2) (layer "F.Cu") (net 13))
 (segment (start 158.00415 107.5) (end 162.382 103.12215) (width 0.2) (layer "F.Cu") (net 13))
 (segment (start 159.63005 93.36995) (end 159.86995 93.36995) (width 0.2) (layer "F.Cu") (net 13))
 (segment (start 159.86995 93.36995) (end 161.5 95) (width 0.2) (layer "F.Cu") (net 13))
 (segment (start 159.19 82.685) (end 146.49 82.685) (width 0.2) (layer "F.Cu") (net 16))
 (segment (start 179.51 90.305) (end 179.51 82.685) (width 0.2) (layer "F.Cu") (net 15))
 (segment (start 179.51 82.685) (end 169.35 82.685) (width 0.2) (layer "F.Cu") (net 15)))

